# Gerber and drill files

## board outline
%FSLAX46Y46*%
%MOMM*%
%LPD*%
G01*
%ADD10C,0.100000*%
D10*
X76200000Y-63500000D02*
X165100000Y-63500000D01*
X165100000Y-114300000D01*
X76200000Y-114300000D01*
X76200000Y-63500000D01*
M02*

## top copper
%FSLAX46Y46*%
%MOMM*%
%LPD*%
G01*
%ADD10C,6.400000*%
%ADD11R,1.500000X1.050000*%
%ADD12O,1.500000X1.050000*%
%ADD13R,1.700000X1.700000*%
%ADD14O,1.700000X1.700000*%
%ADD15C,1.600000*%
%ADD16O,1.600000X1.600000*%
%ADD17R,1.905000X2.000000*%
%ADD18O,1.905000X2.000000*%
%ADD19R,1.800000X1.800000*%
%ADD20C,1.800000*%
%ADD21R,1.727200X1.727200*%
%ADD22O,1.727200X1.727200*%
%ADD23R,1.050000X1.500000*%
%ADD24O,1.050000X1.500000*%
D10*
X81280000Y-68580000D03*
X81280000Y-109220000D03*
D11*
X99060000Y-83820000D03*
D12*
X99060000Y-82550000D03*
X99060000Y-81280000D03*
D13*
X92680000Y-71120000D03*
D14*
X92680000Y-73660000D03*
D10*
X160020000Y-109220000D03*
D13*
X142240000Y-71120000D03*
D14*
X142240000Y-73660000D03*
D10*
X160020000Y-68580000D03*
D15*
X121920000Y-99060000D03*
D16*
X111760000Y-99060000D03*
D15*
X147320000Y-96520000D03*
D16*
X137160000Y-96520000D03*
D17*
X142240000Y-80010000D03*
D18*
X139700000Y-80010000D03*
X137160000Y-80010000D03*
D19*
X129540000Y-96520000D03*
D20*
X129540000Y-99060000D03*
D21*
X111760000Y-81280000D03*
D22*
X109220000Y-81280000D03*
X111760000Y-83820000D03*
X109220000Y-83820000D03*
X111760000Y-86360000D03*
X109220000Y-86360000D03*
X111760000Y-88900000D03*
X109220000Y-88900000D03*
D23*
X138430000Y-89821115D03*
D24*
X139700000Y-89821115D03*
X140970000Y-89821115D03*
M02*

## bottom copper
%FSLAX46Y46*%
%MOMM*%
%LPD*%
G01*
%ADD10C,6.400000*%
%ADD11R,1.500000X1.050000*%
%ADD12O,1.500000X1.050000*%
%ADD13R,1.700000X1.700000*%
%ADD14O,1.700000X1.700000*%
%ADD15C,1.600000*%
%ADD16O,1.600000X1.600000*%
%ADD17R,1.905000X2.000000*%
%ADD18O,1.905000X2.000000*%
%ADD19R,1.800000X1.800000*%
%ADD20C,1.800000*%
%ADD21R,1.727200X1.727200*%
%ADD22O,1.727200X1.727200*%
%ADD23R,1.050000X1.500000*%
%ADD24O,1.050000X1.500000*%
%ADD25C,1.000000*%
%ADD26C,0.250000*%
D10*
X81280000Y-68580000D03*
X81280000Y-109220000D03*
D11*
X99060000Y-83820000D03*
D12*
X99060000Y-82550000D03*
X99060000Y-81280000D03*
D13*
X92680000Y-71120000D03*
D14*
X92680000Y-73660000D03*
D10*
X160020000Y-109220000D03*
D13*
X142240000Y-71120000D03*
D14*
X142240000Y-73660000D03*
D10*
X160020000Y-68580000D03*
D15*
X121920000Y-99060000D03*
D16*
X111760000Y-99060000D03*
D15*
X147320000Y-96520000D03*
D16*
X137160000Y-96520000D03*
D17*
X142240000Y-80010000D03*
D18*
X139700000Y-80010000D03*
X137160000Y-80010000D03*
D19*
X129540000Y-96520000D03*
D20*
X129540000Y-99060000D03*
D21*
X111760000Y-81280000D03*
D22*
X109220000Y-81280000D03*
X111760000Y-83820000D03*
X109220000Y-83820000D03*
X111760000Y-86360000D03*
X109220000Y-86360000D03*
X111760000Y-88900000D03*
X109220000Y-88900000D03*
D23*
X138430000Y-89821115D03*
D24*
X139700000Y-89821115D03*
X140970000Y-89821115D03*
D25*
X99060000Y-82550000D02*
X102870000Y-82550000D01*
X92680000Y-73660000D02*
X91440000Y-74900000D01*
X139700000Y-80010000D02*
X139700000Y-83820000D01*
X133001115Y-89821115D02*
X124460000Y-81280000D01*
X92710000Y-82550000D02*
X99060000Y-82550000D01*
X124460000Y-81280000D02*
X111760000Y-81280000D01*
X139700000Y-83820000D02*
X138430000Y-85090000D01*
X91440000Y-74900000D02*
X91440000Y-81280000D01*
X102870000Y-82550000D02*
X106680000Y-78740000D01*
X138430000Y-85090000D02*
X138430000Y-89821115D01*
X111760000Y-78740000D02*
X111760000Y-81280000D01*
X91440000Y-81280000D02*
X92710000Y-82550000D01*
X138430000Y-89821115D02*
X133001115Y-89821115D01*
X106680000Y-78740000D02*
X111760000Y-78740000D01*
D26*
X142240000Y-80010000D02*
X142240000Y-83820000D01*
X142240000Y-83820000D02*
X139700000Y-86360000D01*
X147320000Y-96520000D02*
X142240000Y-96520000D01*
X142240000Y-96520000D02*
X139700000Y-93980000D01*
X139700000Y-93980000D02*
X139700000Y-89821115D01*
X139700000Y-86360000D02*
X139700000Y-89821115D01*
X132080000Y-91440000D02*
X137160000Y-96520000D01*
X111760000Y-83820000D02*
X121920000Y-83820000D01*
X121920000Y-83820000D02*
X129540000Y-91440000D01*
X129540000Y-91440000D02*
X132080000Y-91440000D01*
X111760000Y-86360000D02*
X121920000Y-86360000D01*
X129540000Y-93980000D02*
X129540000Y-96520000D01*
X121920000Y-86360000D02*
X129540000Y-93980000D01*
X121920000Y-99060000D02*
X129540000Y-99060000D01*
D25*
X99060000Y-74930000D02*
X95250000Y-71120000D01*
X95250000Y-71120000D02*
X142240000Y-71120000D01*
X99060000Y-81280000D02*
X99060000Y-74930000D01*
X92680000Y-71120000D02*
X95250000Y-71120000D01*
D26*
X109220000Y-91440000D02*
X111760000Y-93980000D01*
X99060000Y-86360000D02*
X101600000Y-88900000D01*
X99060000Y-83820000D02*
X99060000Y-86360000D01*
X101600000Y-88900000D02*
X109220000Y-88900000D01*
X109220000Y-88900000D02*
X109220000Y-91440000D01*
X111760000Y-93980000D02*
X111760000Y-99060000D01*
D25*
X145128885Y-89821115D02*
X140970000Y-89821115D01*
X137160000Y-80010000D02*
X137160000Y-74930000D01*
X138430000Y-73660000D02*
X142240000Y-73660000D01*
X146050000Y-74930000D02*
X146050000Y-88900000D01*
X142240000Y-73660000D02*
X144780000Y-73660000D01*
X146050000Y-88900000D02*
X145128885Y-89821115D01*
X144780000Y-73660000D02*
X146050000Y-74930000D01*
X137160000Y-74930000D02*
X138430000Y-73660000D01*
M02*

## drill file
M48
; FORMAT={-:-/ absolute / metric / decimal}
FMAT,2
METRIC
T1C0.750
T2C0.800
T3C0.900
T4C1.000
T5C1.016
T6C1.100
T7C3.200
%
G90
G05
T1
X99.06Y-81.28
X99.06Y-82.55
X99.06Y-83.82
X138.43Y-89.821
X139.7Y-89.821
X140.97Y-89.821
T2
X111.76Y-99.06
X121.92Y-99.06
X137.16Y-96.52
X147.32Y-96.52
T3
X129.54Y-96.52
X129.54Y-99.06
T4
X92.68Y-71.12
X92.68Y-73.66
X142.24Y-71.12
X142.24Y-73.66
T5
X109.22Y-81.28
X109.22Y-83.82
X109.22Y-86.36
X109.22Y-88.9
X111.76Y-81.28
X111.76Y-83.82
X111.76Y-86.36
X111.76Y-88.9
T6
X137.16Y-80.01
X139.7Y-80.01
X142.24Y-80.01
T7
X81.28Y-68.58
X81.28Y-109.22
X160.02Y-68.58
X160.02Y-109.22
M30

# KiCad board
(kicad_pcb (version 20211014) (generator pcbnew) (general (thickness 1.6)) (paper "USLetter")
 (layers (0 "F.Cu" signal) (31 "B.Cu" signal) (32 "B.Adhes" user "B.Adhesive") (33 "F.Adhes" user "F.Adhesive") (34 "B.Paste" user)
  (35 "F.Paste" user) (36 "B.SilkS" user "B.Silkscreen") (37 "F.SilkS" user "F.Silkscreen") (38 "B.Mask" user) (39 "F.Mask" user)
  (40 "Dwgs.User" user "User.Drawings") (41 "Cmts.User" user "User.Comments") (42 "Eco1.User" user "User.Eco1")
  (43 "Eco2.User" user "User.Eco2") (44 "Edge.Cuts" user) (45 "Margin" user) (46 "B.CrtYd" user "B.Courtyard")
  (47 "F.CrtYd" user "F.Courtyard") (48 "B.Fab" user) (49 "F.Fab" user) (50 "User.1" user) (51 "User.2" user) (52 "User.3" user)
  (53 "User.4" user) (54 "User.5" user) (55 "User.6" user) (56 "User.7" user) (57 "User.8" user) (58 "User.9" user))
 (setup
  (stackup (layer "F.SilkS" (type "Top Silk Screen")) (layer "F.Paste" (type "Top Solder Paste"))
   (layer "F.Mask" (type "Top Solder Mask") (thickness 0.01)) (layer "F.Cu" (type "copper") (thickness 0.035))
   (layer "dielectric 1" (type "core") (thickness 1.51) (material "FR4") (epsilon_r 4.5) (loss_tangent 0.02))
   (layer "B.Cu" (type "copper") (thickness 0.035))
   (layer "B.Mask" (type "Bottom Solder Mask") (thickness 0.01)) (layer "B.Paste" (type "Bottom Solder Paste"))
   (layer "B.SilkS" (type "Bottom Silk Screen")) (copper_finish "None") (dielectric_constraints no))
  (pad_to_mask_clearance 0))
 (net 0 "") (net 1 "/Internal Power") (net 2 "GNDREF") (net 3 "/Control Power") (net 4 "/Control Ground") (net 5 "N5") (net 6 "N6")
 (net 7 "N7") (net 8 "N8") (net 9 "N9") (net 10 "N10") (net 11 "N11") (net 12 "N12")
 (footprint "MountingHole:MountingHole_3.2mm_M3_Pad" (layer "F.Cu") (at 81.28 68.58)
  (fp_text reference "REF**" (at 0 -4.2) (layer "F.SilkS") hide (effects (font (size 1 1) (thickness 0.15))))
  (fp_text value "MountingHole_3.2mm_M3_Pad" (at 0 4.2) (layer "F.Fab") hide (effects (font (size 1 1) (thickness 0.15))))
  (pad "1" thru_hole circle (at 0 0) (size 6.4 6.4) (drill 3.2) (layers *.Cu *.Mask)))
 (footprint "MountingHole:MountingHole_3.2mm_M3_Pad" (layer "F.Cu") (at 81.28 109.22)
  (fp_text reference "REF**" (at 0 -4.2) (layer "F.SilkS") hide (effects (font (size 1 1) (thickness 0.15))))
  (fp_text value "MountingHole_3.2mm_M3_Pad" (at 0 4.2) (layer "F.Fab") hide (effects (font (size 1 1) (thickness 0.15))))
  (pad "1" thru_hole circle (at 0 0) (size 6.4 6.4) (drill 3.2) (layers *.Cu *.Mask)))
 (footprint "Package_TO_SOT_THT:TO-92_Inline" (layer "F.Cu") (at 99.06 83.82 90)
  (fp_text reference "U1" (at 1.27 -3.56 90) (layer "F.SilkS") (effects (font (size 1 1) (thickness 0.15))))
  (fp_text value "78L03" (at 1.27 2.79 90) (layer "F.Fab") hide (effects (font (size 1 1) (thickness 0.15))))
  (pad "1" thru_hole rect (at 0 0 90) (size 1.05 1.5) (drill 0.75) (layers *.Cu *.Mask) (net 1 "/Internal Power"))
  (pad "2" thru_hole oval (at 1.27 0 90) (size 1.05 1.5) (drill 0.75) (layers *.Cu *.Mask) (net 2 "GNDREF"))
  (pad "3" thru_hole oval (at 2.54 0 90) (size 1.05 1.5) (drill 0.75) (layers *.Cu *.Mask) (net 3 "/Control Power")))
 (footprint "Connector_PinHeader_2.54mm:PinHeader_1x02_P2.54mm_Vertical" (layer "F.Cu") (at 92.68 71.12)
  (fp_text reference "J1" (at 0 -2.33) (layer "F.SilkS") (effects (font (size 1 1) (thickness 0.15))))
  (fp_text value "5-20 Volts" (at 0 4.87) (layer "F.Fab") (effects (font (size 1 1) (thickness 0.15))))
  (pad "1" thru_hole rect (at 0 0) (size 1.7 1.7) (drill 1) (layers *.Cu *.Mask) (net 3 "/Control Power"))
  (pad "2" thru_hole oval (at 0 2.54) (size 1.7 1.7) (drill 1) (layers *.Cu *.Mask) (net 2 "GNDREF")))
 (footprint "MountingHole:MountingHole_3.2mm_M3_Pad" (layer "F.Cu") (at 160.02 109.22)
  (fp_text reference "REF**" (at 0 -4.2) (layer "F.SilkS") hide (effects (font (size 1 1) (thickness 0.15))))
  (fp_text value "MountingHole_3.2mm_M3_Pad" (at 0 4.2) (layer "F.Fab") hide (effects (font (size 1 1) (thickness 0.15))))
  (pad "1" thru_hole circle (at 0 0) (size 6.4 6.4) (drill 3.2) (layers *.Cu *.Mask)))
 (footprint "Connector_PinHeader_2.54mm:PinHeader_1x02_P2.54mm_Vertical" (layer "F.Cu") (at 142.24 71.12)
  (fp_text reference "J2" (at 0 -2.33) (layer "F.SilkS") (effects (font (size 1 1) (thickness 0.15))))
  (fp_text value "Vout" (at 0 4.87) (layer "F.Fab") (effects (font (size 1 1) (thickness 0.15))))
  (pad "1" thru_hole rect (at 0 0) (size 1.7 1.7) (drill 1) (layers *.Cu *.Mask) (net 3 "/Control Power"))
  (pad "2" thru_hole oval (at 0 2.54) (size 1.7 1.7) (drill 1) (layers *.Cu *.Mask) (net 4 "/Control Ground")))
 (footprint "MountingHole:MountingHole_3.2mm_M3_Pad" (layer "F.Cu") (at 160.02 68.58)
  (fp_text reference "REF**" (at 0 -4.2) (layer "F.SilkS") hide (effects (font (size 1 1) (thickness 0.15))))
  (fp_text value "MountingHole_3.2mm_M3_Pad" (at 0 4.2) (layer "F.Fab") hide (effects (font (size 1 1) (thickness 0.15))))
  (pad "1" thru_hole circle (at 0 0) (size 6.4 6.4) (drill 3.2) (layers *.Cu *.Mask)))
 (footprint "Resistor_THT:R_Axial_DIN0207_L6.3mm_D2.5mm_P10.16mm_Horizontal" (layer "F.Cu") (at 121.92 99.06 180)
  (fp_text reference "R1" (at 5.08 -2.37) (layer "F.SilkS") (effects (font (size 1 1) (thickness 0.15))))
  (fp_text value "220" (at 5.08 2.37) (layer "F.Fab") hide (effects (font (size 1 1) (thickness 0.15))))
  (pad "1" thru_hole circle (at 0 0 180) (size 1.6 1.6) (drill 0.8) (layers *.Cu *.Mask) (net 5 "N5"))
  (pad "2" thru_hole oval (at 10.16 0 180) (size 1.6 1.6) (drill 0.8) (layers *.Cu *.Mask) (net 1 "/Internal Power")))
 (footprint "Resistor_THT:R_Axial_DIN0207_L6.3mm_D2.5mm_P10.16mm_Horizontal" (layer "F.Cu") (at 147.32 96.52 180)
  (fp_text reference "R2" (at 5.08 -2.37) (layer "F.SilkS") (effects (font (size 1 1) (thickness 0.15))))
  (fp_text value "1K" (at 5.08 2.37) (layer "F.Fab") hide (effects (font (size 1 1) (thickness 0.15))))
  (pad "1" thru_hole circle (at 0 0 180) (size 1.6 1.6) (drill 0.8) (layers *.Cu *.Mask) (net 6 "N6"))
  (pad "2" thru_hole oval (at 10.16 0 180) (size 1.6 1.6) (drill 0.8) (layers *.Cu *.Mask) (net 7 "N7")))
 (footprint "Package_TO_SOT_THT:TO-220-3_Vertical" (layer "F.Cu") (at 142.24 80.01 180)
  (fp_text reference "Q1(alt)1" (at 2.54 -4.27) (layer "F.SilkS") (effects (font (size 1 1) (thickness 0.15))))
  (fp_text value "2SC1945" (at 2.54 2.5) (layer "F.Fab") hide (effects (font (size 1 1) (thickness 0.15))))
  (pad "1" thru_hole rect (at 0 0 180) (size 1.905 2) (drill 1.1) (layers *.Cu *.Mask) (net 6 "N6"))
  (pad "2" thru_hole oval (at 2.54 0 180) (size 1.905 2) (drill 1.1) (layers *.Cu *.Mask) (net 2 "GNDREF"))
  (pad "3" thru_hole oval (at 5.08 0 180) (size 1.905 2) (drill 1.1) (layers *.Cu *.Mask) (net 4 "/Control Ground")))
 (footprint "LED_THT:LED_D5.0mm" (layer "F.Cu") (at 129.54 96.52 -90)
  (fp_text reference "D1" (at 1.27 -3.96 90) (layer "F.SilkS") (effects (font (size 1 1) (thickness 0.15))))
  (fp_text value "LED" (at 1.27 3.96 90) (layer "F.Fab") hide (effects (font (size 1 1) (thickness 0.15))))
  (pad "1" thru_hole rect (at 0 0 270) (size 1.8 1.8) (drill 0.9) (layers *.Cu *.Mask) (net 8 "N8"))
  (pad "2" thru_hole circle (at 2.54 0 270) (size 1.8 1.8) (drill 0.9) (layers *.Cu *.Mask) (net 5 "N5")))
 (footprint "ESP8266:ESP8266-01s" (layer "F.Cu") (at 109.22 81.28)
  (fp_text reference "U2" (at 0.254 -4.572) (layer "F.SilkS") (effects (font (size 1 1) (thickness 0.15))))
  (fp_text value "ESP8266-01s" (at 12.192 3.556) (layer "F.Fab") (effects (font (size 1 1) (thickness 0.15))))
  (pad "1" thru_hole rect (at 2.54 0) (size 1.7272 1.7272) (drill 1.016) (layers *.Cu *.Mask "F.SilkS") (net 2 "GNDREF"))
  (pad "2" thru_hole oval (at 0 0) (size 1.7272 1.7272) (drill 1.016) (layers *.Cu *.Mask "F.SilkS") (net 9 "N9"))
  (pad "3" thru_hole oval (at 2.54 2.54) (size 1.7272 1.7272) (drill 1.016) (layers *.Cu *.Mask "F.SilkS") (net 7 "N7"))
  (pad "4" thru_hole oval (at 0 2.54) (size 1.7272 1.7272) (drill 1.016) (layers *.Cu *.Mask "F.SilkS") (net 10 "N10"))
  (pad "5" thru_hole oval (at 2.54 5.08) (size 1.7272 1.7272) (drill 1.016) (layers *.Cu *.Mask "F.SilkS") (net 8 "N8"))
  (pad "6" thru_hole oval (at 0 5.08) (size 1.7272 1.7272) (drill 1.016) (layers *.Cu *.Mask "F.SilkS") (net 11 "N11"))
  (pad "7" thru_hole oval (at 2.54 7.62) (size 1.7272 1.7272) (drill 1.016) (layers *.Cu *.Mask "F.SilkS") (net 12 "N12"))
  (pad "8" thru_hole oval (at 0 7.62) (size 1.7272 1.7272) (drill 1.016) (layers *.Cu *.Mask "F.SilkS") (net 1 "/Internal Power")))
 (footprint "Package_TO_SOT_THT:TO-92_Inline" (layer "F.Cu") (at 138.43 89.821115)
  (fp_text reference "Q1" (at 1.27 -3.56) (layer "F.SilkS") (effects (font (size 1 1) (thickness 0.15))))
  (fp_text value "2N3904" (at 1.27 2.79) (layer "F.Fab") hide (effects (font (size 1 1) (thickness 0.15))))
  (pad "1" thru_hole rect (at 0 0) (size 1.05 1.5) (drill 0.75) (layers *.Cu *.Mask) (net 2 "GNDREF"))
  (pad "2" thru_hole oval (at 1.27 0) (size 1.05 1.5) (drill 0.75) (layers *.Cu *.Mask) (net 6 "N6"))
  (pad "3" thru_hole oval (at 2.54 0) (size 1.05 1.5) (drill 0.75) (layers *.Cu *.Mask) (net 4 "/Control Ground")))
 (gr_rect (start 76.2 63.5) (end 165.1 114.3) (layer "Edge.Cuts") (width 0.1) (fill none))
 (segment (start 99.06 82.55) (end 102.87 82.55) (width 1) (layer "B.Cu") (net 2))
 (segment (start 92.68 73.66) (end 91.44 74.9) (width 1) (layer "B.Cu") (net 2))
 (segment (start 139.7 80.01) (end 139.7 83.82) (width 1) (layer "B.Cu") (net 2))
 (segment (start 133.001115 89.821115) (end 124.46 81.28) (width 1) (layer "B.Cu") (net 2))
 (segment (start 92.71 82.55) (end 99.06 82.55) (width 1) (layer "B.Cu") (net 2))
 (segment (start 124.46 81.28) (end 111.76 81.28) (width 1) (layer "B.Cu") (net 2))
 (segment (start 139.7 83.82) (end 138.43 85.09) (width 1) (layer "B.Cu") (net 2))
 (segment (start 91.44 74.9) (end 91.44 81.28) (width 1) (layer "B.Cu") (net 2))
 (segment (start 102.87 82.55) (end 106.68 78.74) (width 1) (layer "B.Cu") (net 2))
 (segment (start 138.43 85.09) (end 138.43 89.821115) (width 1) (layer "B.Cu") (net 2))
 (segment (start 111.76 78.74) (end 111.76 81.28) (width 1) (layer "B.Cu") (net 2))
 (segment (start 91.44 81.28) (end 92.71 82.55) (width 1) (layer "B.Cu") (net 2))
 (segment (start 138.43 89.821115) (end 133.001115 89.821115) (width 1) (layer "B.Cu") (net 2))
 (segment (start 106.68 78.74) (end 111.76 78.74) (width 1) (layer "B.Cu") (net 2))
 (segment (start 142.24 80.01) (end 142.24 83.82) (width 0.25) (layer "B.Cu") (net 6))
 (segment (start 142.24 83.82) (end 139.7 86.36) (width 0.25) (layer "B.Cu") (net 6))
 (segment (start 147.32 96.52) (end 142.24 96.52) (width 0.25) (layer "B.Cu") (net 6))
 (segment (start 142.24 96.52) (end 139.7 93.98) (width 0.25) (layer "B.Cu") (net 6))
 (segment (start 139.7 93.98) (end 139.7 89.821115) (width 0.25) (layer "B.Cu") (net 6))
 (segment (start 139.7 86.36) (end 139.7 89.821115) (width 0.25) (layer "B.Cu") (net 6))
 (segment (start 132.08 91.44) (end 137.16 96.52) (width 0.25) (layer "B.Cu") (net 7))
 (segment (start 111.76 83.82) (end 121.92 83.82) (width 0.25) (layer "B.Cu") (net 7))
 (segment (start 121.92 83.82) (end 129.54 91.44) (width 0.25) (layer "B.Cu") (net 7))
 (segment (start 129.54 91.44) (end 132.08 91.44) (width 0.25) (layer "B.Cu") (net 7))
 (segment (start 111.76 86.36) (end 121.92 86.36) (width 0.25) (layer "B.Cu") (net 8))
 (segment (start 129.54 93.98) (end 129.54 96.52) (width 0.25) (layer "B.Cu") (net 8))
 (segment (start 121.92 86.36) (end 129.54 93.98) (width 0.25) (layer "B.Cu") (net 8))
 (segment (start 121.92 99.06) (end 129.54 99.06) (width 0.25) (layer "B.Cu") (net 5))
 (segment (start 99.06 74.93) (end 95.25 71.12) (width 1) (layer "B.Cu") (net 3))
 (segment (start 95.25 71.12) (end 142.24 71.12) (width 1) (layer "B.Cu") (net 3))
 (segment (start 99.06 81.28) (end 99.06 74.93) (width 1) (layer "B.Cu") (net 3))
 (segment (start 92.68 71.12) (end 95.25 71.12) (width 1) (layer "B.Cu") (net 3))
 (segment (start 109.22 91.44) (end 111.76 93.98) (width 0.25) (layer "B.Cu") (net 1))
 (segment (start 99.06 86.36) (end 101.6 88.9) (width 0.25) (layer "B.Cu") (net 1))
 (segment (start 99.06 83.82) (end 99.06 86.36) (width 0.25) (layer "B.Cu") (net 1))
 (segment (start 101.6 88.9) (end 109.22 88.9) (width 0.25) (layer "B.Cu") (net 1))
 (segment (start 109.22 88.9) (end 109.22 91.44) (width 0.25) (layer "B.Cu") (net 1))
 (segment (start 111.76 93.98) (end 111.76 99.06) (width 0.25) (layer "B.Cu") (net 1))
 (segment (start 145.128885 89.821115) (end 140.97 89.821115) (width 1) (layer "B.Cu") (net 4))
 (segment (start 137.16 80.01) (end 137.16 74.93) (width 1) (layer "B.Cu") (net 4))
 (segment (start 138.43 73.66) (end 142.24 73.66) (width 1) (layer "B.Cu") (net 4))
 (segment (start 146.05 74.93) (end 146.05 88.9) (width 1) (layer "B.Cu") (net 4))
 (segment (start 142.24 73.66) (end 144.78 73.66) (width 1) (layer "B.Cu") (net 4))
 (segment (start 146.05 88.9) (end 145.128885 89.821115) (width 1) (layer "B.Cu") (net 4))
 (segment (start 144.78 73.66) (end 146.05 74.93) (width 1) (layer "B.Cu") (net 4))
 (segment (start 137.16 74.93) (end 138.43 73.66) (width 1) (layer "B.Cu") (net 4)))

